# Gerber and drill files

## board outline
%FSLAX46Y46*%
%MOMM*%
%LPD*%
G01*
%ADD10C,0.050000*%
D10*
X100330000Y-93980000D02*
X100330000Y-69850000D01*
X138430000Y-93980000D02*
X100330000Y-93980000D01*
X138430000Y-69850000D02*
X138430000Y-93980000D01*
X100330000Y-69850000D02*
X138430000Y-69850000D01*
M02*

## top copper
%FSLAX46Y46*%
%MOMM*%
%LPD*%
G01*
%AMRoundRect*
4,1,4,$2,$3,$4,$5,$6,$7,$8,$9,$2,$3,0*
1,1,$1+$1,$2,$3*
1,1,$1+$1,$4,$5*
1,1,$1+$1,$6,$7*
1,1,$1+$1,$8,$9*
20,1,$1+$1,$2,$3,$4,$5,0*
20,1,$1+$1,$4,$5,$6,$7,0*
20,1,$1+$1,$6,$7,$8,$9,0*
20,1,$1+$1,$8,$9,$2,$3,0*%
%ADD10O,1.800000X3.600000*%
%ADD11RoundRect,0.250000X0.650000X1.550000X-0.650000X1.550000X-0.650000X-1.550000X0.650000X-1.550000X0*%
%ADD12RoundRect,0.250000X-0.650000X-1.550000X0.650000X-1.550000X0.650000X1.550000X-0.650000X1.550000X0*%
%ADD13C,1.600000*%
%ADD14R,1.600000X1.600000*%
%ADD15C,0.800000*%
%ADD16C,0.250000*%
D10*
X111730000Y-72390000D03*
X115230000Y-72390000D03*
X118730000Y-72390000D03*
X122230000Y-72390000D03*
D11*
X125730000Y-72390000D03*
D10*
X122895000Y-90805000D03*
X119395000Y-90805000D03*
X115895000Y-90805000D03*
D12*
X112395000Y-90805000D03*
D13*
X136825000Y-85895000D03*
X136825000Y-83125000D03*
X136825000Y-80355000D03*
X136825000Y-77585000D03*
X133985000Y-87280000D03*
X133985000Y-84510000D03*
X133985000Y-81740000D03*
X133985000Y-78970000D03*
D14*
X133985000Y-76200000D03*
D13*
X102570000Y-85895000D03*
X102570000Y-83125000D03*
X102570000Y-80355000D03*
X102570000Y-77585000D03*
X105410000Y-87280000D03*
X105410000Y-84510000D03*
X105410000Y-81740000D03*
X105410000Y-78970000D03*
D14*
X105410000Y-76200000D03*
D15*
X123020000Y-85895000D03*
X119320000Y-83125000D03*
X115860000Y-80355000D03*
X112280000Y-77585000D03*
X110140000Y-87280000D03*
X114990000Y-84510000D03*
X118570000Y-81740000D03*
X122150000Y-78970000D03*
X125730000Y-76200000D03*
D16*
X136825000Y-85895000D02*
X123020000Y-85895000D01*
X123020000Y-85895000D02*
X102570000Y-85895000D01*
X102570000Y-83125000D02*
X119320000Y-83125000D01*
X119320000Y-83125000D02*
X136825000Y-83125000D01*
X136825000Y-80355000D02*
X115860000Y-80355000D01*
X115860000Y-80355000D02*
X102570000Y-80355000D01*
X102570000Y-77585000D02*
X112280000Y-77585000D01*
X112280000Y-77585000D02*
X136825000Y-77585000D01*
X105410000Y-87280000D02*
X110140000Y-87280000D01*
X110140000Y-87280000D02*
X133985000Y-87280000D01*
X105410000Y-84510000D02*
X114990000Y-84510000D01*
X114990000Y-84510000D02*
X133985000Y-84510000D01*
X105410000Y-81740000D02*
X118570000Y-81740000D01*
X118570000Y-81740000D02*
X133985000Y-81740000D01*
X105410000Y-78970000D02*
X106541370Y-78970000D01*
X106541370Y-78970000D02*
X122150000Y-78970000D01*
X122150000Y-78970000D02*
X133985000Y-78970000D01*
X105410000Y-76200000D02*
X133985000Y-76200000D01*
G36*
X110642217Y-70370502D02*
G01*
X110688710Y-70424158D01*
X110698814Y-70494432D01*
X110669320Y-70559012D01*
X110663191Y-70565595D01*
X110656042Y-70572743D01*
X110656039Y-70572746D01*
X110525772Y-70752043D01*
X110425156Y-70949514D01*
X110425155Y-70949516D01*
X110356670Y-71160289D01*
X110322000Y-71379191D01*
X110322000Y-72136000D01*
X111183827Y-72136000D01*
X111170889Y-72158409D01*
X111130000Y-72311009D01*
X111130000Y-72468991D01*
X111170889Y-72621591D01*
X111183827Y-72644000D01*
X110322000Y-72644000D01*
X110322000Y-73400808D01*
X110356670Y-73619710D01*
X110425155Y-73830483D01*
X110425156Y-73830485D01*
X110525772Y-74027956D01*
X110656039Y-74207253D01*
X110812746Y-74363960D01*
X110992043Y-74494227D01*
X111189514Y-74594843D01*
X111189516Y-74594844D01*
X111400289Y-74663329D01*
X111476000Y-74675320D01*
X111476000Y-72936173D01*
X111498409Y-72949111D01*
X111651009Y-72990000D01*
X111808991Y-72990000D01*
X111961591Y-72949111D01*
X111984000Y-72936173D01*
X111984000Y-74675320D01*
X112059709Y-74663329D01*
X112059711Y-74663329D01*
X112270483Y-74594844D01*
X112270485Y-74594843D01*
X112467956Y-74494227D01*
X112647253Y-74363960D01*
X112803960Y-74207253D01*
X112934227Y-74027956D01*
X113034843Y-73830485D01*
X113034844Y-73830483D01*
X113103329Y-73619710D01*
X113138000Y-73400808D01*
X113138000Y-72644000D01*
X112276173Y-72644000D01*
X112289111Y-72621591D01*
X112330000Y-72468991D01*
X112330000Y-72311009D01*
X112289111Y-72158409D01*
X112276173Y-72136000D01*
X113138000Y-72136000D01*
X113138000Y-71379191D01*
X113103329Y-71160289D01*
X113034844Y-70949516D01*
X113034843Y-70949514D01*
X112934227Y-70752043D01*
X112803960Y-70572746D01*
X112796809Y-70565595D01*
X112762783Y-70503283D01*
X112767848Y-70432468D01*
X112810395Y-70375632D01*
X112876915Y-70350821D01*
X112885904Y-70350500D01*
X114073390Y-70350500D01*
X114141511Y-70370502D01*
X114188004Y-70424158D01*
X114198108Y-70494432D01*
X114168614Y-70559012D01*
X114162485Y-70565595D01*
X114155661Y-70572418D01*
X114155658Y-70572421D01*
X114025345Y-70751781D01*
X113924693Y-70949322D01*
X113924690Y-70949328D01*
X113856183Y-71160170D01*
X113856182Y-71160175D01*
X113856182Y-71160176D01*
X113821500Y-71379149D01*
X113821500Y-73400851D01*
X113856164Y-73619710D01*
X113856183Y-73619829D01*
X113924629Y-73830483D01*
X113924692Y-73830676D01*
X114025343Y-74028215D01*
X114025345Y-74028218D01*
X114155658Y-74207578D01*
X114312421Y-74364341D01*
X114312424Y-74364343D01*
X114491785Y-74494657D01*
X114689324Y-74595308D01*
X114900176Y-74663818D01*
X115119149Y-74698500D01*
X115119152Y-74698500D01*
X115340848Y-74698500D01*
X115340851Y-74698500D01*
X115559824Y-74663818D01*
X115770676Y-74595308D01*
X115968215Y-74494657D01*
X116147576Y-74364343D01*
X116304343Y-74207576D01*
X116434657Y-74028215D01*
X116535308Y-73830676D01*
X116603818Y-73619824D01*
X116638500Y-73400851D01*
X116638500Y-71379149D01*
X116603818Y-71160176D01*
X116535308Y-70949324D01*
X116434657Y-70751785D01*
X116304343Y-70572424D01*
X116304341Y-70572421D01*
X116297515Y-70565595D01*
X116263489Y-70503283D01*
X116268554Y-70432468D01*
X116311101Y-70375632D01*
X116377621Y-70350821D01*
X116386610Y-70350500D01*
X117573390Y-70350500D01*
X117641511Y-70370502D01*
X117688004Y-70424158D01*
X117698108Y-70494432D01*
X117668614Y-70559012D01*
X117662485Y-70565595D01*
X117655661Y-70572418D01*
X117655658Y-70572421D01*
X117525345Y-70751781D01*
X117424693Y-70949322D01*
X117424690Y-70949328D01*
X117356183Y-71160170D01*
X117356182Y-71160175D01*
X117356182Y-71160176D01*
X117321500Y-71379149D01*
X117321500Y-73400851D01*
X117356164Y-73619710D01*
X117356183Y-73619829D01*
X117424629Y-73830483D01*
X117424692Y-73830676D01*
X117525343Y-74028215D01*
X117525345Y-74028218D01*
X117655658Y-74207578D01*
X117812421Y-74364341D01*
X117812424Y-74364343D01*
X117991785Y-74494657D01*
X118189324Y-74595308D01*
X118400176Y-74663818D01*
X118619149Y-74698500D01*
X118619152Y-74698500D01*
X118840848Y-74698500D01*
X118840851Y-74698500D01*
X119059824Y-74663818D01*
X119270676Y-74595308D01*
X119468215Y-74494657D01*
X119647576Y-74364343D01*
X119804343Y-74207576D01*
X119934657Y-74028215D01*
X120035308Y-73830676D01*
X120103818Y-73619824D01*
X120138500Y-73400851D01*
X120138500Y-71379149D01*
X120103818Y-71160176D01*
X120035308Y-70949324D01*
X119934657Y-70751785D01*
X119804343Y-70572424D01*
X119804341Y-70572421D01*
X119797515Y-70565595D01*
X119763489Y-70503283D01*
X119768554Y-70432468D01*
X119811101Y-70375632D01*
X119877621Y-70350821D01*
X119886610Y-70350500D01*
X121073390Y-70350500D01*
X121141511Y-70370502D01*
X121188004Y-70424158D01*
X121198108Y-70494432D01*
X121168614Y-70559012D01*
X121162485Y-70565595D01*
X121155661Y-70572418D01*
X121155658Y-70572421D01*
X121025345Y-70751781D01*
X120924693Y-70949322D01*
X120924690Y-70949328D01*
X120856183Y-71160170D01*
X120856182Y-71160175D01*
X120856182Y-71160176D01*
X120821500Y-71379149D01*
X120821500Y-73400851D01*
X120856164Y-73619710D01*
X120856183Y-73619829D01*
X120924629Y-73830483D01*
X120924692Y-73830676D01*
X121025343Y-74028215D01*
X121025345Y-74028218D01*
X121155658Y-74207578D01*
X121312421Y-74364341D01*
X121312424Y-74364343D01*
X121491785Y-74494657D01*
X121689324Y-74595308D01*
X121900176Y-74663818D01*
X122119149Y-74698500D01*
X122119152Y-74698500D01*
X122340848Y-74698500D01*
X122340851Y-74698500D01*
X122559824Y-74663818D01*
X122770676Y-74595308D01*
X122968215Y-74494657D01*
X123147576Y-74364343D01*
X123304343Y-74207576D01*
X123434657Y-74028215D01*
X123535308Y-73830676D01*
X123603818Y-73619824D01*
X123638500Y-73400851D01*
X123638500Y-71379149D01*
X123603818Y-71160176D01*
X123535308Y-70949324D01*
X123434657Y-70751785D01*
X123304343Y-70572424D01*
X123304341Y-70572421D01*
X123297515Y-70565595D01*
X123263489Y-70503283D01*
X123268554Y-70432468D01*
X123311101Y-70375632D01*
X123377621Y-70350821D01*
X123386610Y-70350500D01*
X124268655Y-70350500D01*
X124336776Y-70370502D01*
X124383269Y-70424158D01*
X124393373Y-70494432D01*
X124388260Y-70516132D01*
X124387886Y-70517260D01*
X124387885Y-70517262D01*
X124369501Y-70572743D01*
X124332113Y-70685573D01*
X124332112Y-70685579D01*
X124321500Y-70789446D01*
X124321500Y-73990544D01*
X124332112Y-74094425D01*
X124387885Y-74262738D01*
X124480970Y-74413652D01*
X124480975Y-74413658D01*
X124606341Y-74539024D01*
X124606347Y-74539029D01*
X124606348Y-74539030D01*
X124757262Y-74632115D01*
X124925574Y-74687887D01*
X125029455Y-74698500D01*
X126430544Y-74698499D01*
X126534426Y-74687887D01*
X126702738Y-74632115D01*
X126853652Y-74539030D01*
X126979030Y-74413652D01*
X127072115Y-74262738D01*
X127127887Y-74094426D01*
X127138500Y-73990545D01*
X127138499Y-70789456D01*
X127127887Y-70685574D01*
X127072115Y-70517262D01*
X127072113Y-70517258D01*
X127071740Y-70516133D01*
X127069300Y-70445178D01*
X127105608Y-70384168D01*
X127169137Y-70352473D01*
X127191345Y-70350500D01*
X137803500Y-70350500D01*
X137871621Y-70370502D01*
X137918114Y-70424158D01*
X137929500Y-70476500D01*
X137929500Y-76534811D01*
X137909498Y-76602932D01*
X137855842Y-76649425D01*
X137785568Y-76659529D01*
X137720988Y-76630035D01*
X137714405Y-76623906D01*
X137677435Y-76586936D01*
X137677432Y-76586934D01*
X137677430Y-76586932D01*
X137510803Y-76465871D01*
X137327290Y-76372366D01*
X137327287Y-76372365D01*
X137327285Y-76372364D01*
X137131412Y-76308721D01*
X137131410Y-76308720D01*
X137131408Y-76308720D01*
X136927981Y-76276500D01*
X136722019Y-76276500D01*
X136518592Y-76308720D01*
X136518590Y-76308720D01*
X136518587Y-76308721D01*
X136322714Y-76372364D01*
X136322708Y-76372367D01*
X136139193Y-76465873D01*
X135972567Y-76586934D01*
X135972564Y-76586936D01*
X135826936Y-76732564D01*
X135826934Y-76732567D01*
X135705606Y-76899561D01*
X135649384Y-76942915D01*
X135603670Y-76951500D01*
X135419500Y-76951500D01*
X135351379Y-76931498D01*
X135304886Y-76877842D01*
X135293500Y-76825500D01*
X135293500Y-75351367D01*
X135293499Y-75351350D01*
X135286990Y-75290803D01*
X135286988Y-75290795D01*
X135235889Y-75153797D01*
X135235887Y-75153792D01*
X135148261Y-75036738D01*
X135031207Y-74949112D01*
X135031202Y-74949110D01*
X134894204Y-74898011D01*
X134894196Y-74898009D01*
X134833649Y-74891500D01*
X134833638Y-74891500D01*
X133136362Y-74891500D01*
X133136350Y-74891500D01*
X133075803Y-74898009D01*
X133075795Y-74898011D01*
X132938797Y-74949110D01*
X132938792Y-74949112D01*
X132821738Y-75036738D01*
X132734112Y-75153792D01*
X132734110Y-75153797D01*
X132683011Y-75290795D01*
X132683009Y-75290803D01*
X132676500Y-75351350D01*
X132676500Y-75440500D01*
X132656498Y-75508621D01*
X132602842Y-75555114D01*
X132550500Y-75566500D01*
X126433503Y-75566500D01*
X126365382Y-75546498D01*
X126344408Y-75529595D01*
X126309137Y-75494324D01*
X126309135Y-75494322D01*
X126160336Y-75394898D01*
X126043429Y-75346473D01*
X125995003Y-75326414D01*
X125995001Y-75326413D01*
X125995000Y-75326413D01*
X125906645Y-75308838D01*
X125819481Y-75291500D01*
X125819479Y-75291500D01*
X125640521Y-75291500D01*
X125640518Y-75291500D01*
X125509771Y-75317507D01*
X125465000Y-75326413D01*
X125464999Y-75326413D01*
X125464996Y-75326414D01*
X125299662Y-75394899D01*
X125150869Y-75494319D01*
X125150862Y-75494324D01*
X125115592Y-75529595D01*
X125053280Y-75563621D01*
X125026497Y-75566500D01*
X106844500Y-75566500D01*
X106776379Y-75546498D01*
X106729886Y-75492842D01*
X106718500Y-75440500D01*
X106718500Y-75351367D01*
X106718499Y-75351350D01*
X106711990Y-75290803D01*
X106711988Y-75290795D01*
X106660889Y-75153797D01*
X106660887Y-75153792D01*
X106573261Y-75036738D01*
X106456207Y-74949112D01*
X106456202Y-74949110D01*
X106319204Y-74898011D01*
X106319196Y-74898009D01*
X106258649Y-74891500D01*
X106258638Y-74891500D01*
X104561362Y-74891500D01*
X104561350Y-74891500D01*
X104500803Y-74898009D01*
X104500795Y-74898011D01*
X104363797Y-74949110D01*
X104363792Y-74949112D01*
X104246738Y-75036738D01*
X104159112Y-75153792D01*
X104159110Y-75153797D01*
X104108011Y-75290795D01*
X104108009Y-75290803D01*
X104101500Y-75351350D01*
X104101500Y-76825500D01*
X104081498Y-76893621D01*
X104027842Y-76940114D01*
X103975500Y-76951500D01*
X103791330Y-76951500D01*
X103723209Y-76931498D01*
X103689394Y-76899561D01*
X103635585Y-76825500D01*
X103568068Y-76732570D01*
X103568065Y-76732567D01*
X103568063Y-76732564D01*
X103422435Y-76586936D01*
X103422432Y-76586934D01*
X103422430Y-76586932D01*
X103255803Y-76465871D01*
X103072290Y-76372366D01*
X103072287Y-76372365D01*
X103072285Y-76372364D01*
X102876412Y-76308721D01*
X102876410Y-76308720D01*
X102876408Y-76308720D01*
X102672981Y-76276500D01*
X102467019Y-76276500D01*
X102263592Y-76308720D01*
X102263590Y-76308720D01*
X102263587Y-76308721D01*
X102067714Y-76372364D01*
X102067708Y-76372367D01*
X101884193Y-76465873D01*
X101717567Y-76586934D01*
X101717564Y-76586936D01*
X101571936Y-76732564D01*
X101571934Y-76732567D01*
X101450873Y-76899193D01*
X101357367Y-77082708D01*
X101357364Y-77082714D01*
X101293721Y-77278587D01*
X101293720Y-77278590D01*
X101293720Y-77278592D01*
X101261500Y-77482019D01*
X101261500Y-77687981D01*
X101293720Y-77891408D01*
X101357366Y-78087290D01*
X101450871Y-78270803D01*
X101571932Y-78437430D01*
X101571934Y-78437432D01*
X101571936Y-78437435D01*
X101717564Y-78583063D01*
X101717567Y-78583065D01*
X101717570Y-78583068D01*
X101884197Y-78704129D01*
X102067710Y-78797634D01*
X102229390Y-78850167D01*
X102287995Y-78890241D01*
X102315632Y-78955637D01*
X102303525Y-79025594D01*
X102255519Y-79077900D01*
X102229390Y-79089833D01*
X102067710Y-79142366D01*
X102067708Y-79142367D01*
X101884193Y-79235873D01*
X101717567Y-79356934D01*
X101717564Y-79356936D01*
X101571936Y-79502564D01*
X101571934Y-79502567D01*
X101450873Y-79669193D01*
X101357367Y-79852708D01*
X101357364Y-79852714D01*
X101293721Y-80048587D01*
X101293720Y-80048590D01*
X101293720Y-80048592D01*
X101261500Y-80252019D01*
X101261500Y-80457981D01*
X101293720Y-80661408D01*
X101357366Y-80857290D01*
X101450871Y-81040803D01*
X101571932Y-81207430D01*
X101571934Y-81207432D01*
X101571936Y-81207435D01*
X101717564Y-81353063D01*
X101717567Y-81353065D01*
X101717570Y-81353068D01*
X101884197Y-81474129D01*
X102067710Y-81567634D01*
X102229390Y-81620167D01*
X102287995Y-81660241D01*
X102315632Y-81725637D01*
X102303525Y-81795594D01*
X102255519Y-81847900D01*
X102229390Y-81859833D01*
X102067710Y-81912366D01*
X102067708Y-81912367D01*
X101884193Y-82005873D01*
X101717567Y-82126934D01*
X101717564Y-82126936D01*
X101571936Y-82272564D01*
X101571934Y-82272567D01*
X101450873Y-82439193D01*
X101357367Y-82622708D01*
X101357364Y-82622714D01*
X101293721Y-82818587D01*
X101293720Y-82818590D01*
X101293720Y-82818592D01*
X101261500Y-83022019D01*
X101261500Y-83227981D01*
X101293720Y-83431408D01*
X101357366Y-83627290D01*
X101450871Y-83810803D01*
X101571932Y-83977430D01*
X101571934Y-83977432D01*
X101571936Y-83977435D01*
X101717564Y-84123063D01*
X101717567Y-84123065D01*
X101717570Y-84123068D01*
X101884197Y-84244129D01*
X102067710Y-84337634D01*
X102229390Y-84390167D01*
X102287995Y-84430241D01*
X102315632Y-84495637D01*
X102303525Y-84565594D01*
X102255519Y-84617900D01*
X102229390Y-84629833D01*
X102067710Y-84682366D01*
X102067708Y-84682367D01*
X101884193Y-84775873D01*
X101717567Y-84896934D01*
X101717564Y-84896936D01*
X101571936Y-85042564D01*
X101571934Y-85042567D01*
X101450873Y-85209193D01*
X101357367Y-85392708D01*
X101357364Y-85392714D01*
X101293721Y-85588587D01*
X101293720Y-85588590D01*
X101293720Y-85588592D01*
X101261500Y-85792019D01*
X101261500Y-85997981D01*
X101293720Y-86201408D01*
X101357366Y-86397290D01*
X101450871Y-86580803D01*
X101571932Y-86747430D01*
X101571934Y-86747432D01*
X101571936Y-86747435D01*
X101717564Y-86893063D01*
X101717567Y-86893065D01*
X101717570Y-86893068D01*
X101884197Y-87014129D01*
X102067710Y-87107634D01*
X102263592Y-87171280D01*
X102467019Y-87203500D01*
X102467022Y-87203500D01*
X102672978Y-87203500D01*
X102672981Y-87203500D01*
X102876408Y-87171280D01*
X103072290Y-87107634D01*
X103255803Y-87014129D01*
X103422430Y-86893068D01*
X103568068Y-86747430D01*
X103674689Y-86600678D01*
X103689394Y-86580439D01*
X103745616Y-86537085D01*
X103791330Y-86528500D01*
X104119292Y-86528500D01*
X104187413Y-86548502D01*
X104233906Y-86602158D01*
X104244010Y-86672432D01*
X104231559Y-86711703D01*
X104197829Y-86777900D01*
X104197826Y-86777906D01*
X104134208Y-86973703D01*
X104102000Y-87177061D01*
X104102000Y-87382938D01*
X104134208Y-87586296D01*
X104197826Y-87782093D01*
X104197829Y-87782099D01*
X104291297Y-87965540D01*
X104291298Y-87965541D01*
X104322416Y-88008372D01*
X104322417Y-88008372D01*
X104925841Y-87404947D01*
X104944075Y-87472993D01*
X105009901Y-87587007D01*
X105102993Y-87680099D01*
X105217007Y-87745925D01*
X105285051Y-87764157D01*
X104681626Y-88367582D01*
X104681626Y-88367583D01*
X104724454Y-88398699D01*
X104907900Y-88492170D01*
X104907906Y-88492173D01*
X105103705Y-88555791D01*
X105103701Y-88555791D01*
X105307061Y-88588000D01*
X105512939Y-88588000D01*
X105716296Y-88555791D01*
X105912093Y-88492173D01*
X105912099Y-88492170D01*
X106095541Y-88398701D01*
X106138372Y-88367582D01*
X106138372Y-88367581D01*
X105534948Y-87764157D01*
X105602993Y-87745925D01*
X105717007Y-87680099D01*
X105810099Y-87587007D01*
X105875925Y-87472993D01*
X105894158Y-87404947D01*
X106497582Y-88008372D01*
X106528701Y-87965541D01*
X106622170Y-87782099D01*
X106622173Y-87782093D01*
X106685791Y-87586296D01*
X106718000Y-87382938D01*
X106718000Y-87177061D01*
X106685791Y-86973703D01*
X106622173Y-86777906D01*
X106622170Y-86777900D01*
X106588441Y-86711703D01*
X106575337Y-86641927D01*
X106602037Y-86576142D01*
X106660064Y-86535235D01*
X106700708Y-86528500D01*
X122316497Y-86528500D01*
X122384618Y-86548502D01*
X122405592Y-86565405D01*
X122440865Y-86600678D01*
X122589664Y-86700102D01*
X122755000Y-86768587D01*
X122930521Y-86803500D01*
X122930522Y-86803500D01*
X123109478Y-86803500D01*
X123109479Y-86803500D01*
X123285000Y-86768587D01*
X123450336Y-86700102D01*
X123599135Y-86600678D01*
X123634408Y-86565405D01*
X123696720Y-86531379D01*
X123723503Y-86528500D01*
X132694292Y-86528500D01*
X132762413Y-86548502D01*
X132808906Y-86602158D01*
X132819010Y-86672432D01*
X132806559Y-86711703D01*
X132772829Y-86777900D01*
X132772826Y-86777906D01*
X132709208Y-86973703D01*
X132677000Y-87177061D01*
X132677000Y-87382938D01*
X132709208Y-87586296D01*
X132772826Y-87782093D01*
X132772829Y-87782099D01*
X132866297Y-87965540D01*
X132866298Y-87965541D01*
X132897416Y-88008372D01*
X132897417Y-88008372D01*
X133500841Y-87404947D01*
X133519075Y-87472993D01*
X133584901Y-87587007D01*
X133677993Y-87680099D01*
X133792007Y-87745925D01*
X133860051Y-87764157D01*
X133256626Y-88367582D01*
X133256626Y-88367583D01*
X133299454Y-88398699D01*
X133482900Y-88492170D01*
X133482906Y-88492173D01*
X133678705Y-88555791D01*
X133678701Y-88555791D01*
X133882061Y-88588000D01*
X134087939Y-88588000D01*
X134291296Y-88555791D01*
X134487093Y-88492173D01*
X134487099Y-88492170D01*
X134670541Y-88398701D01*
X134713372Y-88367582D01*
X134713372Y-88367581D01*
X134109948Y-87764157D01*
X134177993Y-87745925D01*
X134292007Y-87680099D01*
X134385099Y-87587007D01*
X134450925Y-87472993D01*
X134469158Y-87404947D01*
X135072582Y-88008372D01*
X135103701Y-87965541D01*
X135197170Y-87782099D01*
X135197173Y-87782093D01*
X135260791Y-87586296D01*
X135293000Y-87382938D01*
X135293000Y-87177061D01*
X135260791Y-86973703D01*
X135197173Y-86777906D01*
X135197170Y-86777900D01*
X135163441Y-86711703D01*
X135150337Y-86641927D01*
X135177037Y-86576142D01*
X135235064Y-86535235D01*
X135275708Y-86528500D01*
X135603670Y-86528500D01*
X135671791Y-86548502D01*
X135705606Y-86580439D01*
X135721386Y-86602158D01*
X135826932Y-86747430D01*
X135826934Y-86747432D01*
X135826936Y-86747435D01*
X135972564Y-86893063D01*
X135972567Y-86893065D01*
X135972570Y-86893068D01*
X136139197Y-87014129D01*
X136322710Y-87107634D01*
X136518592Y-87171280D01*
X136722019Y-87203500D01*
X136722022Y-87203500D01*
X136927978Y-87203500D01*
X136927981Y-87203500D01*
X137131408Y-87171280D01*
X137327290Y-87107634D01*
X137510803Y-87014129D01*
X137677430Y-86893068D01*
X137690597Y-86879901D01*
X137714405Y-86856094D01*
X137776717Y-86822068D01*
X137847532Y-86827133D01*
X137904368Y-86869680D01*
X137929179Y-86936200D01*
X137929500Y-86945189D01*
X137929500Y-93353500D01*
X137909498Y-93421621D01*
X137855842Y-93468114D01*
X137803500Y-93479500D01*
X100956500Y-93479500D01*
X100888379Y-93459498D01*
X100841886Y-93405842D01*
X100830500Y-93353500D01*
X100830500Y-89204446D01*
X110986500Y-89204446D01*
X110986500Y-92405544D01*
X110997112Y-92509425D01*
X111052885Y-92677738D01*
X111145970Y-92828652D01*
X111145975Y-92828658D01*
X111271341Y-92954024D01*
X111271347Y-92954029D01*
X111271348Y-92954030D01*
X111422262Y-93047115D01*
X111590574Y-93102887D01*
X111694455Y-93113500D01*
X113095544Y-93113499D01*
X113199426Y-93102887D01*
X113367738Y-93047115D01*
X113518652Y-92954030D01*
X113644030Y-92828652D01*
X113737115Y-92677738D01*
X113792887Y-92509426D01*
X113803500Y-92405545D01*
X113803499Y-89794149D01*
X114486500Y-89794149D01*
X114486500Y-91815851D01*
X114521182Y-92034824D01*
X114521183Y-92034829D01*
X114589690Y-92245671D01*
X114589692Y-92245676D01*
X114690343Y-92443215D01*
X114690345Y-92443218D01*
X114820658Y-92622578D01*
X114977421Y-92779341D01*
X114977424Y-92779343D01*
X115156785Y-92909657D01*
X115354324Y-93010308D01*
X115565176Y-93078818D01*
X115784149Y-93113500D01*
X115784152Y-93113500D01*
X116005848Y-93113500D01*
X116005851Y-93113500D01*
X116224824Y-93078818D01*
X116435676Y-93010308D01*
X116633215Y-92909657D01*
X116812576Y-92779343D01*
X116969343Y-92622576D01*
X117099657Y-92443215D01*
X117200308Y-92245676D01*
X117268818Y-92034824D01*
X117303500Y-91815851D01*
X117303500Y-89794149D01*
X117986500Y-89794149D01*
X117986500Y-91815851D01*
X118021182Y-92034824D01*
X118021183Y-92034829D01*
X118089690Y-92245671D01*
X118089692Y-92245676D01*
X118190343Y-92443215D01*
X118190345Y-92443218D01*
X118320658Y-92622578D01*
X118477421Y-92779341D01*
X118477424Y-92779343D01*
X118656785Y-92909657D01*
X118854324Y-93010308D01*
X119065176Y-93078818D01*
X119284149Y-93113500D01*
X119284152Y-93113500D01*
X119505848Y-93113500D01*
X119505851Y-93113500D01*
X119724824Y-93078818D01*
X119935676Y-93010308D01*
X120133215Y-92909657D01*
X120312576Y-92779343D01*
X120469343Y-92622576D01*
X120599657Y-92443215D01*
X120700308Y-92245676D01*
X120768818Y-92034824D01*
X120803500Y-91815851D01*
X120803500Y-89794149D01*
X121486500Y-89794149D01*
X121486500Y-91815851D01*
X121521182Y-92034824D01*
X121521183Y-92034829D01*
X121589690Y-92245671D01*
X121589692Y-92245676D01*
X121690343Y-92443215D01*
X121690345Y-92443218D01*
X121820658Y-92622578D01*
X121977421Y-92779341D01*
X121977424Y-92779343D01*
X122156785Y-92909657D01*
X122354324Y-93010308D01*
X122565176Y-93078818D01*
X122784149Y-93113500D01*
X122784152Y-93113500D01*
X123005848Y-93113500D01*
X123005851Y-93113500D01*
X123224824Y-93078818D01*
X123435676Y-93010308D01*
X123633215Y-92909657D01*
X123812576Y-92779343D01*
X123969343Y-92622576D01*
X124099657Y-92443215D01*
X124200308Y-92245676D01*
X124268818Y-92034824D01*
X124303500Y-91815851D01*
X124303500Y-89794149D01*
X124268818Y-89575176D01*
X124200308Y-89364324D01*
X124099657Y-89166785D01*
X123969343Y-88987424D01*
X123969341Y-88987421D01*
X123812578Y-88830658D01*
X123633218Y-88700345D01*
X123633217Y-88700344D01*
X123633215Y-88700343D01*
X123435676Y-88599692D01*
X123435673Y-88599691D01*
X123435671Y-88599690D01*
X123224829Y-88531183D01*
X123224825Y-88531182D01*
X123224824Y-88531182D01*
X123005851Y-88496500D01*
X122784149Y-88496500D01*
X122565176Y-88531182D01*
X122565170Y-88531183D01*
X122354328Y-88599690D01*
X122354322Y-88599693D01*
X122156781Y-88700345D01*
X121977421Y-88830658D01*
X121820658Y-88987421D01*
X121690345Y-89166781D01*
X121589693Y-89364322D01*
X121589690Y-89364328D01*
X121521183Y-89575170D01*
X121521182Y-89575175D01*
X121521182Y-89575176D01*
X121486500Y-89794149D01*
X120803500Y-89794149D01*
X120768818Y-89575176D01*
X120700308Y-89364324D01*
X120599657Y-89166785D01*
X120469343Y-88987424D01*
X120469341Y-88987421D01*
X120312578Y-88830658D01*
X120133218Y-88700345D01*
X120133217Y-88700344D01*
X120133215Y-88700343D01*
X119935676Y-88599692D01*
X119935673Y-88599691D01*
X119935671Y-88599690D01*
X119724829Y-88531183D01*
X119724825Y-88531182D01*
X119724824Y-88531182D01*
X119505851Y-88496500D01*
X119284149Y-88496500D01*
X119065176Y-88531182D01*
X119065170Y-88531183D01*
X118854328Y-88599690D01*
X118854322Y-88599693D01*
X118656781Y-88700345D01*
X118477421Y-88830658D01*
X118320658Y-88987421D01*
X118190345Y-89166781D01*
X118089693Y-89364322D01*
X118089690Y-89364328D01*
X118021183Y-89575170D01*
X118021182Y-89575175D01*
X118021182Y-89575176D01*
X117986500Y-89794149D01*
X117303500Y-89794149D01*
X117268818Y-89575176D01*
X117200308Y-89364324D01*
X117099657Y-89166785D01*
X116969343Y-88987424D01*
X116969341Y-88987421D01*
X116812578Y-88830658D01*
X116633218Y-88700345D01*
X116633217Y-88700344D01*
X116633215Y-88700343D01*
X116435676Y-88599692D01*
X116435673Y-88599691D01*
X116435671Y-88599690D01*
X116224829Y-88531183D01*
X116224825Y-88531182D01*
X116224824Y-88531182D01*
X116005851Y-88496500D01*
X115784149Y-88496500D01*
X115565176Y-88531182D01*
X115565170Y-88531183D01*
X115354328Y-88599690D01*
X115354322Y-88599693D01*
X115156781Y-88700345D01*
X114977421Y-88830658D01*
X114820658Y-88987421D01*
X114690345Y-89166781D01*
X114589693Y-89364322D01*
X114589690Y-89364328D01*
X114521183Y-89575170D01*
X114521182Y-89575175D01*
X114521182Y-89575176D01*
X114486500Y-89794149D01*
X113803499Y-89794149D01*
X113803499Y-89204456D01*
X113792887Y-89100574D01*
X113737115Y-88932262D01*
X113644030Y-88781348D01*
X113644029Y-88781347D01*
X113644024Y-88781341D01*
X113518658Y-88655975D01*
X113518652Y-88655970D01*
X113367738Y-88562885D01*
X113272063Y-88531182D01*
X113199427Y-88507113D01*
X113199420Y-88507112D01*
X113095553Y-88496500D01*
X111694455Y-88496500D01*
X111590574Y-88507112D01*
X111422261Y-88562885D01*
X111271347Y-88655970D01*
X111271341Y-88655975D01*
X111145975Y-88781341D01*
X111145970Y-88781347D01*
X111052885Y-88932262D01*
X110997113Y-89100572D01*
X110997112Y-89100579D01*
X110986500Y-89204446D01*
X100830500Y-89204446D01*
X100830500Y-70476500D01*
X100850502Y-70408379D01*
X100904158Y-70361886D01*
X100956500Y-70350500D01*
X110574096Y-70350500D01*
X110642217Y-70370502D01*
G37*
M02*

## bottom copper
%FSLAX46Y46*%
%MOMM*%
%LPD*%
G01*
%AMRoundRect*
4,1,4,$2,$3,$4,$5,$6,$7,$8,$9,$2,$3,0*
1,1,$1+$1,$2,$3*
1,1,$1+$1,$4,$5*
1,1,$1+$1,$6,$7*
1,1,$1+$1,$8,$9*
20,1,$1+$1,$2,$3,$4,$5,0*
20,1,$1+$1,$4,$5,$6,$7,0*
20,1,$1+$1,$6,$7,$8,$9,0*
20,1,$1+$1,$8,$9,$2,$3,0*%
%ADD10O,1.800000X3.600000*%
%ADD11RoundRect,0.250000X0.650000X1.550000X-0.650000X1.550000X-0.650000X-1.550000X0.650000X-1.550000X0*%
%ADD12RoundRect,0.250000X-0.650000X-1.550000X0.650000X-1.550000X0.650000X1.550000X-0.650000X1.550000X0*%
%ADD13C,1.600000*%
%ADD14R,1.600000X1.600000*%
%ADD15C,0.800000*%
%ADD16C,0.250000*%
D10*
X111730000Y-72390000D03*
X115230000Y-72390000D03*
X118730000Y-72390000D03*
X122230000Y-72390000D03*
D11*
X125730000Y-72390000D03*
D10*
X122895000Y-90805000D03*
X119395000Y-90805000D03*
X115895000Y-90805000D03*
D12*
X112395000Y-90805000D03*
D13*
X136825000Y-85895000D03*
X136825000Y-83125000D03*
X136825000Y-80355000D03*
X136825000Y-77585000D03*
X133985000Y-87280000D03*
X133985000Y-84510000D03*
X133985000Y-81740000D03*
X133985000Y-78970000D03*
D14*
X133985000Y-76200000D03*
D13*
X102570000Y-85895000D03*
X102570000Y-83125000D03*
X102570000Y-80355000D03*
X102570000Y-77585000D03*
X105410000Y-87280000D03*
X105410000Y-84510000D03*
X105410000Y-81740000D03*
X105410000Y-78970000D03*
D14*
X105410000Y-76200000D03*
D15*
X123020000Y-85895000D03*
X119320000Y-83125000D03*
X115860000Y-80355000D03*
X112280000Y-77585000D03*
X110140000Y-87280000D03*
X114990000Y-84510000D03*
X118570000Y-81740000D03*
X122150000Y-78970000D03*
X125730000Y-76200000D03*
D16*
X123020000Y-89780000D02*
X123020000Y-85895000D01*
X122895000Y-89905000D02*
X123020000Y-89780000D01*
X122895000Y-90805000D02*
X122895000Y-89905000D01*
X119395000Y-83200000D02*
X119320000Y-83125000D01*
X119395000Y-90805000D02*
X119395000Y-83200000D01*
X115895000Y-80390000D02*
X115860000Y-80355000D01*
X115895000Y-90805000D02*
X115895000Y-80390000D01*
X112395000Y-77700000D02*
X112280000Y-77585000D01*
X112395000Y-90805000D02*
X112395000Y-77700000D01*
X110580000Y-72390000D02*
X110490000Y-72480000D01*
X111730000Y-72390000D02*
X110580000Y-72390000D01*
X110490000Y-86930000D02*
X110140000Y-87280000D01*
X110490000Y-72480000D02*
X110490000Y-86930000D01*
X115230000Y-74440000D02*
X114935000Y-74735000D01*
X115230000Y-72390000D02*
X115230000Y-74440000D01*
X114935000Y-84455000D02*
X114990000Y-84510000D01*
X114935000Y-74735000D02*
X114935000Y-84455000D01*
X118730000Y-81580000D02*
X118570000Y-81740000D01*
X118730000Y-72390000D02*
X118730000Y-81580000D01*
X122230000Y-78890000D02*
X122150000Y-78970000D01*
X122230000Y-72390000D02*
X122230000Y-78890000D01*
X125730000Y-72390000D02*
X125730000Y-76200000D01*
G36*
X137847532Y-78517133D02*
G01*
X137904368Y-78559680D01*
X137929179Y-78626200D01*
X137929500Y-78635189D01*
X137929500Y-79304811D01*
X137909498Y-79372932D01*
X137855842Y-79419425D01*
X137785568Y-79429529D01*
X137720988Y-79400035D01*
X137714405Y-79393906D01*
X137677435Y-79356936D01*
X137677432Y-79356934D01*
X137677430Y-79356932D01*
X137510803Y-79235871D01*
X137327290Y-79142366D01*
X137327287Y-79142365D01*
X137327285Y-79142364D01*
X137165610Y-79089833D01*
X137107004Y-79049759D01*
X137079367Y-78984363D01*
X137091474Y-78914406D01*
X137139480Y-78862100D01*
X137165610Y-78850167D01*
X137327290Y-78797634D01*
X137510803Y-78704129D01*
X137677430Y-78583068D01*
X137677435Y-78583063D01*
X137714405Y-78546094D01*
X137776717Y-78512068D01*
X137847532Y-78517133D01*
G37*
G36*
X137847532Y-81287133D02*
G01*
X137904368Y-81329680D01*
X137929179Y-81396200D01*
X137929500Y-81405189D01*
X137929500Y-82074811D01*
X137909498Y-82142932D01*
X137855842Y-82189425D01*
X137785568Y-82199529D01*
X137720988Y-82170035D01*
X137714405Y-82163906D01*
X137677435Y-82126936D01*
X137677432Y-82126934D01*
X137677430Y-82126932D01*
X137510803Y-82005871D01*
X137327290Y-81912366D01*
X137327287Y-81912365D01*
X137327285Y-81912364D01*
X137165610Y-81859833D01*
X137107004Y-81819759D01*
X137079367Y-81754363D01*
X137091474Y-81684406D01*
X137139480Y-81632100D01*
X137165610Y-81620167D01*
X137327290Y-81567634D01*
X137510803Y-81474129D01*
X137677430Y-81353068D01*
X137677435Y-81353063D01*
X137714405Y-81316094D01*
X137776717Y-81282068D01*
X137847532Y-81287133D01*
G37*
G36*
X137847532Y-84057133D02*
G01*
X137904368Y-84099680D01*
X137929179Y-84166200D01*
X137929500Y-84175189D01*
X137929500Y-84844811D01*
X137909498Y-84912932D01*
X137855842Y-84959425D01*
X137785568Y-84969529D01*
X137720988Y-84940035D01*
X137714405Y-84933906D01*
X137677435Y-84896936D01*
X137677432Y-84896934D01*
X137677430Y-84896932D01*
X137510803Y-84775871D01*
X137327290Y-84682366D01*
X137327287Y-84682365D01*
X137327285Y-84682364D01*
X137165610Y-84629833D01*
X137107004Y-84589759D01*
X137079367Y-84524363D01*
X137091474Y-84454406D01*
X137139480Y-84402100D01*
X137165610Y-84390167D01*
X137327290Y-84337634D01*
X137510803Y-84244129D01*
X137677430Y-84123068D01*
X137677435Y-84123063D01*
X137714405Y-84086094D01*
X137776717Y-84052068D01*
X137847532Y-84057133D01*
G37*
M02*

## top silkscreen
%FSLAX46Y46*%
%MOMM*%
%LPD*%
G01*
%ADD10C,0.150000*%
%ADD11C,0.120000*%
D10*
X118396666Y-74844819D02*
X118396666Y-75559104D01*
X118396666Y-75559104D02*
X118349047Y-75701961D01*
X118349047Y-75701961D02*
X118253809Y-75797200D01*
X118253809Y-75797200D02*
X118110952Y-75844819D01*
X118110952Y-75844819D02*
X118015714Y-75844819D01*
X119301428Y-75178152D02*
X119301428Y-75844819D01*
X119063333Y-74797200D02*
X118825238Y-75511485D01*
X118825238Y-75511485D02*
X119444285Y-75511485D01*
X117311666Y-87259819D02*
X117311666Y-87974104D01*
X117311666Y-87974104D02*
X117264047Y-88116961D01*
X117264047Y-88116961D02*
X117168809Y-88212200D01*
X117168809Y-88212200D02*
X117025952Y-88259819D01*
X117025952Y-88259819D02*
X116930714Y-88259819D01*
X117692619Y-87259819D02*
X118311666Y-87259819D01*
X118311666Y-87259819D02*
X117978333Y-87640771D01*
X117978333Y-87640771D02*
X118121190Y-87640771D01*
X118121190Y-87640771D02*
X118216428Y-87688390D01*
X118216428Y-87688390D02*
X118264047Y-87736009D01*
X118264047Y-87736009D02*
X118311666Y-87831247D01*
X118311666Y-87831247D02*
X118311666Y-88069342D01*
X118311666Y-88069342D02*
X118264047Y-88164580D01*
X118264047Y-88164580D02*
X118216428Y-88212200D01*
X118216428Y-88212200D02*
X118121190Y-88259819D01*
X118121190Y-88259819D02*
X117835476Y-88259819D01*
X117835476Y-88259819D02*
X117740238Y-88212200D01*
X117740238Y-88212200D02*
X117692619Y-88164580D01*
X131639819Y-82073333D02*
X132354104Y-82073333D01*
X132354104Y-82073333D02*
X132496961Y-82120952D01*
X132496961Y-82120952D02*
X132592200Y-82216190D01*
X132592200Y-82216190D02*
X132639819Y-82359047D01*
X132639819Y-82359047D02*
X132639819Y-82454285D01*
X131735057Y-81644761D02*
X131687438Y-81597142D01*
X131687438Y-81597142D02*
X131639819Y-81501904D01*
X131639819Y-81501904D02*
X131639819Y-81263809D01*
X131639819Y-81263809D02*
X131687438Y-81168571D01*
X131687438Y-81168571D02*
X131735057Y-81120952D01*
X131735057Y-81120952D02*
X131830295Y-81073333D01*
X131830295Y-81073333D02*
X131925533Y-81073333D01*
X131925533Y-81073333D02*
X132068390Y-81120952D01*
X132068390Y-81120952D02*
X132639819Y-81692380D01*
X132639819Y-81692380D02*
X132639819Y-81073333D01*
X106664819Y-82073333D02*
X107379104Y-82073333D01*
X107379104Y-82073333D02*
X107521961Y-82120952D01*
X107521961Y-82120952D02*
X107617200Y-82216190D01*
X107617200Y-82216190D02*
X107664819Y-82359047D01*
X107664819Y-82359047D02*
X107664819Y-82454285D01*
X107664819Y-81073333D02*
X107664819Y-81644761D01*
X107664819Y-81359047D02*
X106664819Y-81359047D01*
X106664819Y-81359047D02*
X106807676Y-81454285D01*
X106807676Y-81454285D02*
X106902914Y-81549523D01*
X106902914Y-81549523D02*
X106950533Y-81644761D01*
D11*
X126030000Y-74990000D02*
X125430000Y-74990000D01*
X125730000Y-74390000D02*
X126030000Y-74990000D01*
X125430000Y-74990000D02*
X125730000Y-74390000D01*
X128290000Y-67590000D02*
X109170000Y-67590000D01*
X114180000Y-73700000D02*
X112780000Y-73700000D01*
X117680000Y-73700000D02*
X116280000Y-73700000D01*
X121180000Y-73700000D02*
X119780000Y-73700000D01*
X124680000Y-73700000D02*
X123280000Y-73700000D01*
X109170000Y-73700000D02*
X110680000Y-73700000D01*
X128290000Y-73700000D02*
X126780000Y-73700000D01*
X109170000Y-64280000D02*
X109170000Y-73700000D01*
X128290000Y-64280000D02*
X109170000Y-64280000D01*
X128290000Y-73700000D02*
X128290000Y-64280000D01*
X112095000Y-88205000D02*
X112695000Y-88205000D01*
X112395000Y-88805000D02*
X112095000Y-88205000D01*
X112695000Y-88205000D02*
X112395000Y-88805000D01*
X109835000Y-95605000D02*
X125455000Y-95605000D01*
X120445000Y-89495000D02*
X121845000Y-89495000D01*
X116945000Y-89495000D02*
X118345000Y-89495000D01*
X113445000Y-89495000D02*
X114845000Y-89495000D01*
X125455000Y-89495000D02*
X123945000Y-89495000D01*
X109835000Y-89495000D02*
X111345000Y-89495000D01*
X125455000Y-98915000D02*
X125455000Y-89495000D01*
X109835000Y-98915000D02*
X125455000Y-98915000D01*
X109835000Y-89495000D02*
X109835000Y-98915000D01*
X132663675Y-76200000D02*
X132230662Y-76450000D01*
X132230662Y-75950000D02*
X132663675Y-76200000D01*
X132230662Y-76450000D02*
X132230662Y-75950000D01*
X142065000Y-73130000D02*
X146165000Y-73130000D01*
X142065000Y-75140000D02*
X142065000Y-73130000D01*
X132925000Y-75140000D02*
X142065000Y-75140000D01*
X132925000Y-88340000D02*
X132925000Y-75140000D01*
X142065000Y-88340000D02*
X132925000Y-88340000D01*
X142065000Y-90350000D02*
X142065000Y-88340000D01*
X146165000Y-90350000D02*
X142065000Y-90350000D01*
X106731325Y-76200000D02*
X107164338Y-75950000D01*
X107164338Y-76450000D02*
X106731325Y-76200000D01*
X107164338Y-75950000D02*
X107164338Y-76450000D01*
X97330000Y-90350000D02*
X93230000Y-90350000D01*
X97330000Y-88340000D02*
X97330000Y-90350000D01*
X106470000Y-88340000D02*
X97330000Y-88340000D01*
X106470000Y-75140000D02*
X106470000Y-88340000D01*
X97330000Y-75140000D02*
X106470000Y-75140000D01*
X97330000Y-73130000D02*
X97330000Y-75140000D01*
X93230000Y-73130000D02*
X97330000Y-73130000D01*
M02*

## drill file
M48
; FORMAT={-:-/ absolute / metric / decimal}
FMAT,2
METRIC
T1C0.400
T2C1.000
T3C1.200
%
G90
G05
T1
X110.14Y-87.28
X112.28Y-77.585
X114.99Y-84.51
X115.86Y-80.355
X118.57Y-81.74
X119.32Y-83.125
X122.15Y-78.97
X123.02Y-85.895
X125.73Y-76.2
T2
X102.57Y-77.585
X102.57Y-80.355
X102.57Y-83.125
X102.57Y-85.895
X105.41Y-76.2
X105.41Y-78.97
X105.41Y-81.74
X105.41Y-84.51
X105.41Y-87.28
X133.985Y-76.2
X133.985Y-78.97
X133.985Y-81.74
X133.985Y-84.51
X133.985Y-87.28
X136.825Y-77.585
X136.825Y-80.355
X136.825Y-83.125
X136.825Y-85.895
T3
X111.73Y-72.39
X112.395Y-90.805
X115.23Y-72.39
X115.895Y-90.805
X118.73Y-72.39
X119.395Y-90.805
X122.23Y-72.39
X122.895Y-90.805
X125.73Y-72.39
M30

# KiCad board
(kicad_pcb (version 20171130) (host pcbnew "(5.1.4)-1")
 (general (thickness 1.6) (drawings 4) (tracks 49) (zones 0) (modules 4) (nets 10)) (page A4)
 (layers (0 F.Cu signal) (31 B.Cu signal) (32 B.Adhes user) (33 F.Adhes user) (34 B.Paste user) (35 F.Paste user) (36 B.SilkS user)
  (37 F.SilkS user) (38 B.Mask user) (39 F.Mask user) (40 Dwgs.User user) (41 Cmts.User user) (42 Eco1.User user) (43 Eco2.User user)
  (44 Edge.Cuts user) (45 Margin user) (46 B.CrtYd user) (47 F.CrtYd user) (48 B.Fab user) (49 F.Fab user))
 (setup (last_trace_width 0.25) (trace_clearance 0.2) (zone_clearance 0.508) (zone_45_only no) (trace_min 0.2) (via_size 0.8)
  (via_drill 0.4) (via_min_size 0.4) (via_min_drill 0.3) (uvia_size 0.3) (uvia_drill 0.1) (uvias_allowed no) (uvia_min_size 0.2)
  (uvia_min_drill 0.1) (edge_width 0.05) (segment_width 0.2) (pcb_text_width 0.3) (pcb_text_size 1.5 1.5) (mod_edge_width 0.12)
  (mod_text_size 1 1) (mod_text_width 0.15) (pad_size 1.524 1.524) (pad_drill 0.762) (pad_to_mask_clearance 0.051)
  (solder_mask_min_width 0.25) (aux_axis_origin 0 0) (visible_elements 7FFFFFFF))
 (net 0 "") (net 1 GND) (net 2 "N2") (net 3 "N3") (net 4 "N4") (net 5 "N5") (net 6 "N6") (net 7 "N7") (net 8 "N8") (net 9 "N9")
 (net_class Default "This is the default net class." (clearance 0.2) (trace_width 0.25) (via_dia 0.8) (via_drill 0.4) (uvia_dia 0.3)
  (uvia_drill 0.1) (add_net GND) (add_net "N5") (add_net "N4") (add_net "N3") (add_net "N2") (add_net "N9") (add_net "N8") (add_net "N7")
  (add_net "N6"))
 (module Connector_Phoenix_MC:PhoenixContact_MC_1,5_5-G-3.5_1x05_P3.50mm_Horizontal (layer F.Cu) (at 125.73 72.39 180)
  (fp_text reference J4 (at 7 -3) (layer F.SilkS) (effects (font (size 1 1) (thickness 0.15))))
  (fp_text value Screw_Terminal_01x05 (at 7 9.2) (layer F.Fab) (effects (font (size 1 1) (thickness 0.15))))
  (fp_line (start -0.3 -2.6) (end 0.3 -2.6) (layer F.SilkS) (width 0.12))
  (fp_line (start 0 -2) (end -0.3 -2.6) (layer F.SilkS) (width 0.12))
  (fp_line (start 0.3 -2.6) (end 0 -2) (layer F.SilkS) (width 0.12))
  (fp_line (start -2.56 4.8) (end 16.56 4.8) (layer F.SilkS) (width 0.12))
  (fp_line (start 11.55 -1.31) (end 12.95 -1.31) (layer F.SilkS) (width 0.12))
  (fp_line (start 8.05 -1.31) (end 9.45 -1.31) (layer F.SilkS) (width 0.12))
  (fp_line (start 4.55 -1.31) (end 5.95 -1.31) (layer F.SilkS) (width 0.12))
  (fp_line (start 1.05 -1.31) (end 2.45 -1.31) (layer F.SilkS) (width 0.12))
  (fp_line (start 16.56 -1.31) (end 15.05 -1.31) (layer F.SilkS) (width 0.12))
  (fp_line (start -2.56 -1.31) (end -1.05 -1.31) (layer F.SilkS) (width 0.12))
  (fp_line (start 16.56 8.11) (end 16.56 -1.31) (layer F.SilkS) (width 0.12))
  (fp_line (start -2.56 8.11) (end 16.56 8.11) (layer F.SilkS) (width 0.12))
  (fp_line (start -2.56 -1.31) (end -2.56 8.11) (layer F.SilkS) (width 0.12))
  (pad 5 thru_hole oval (at 14 0 180) (size 1.8 3.6) (drill 1.2) (layers *.Cu *.Mask) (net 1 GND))
  (pad 4 thru_hole oval (at 10.5 0 180) (size 1.8 3.6) (drill 1.2) (layers *.Cu *.Mask) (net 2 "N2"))
  (pad 3 thru_hole oval (at 7 0 180) (size 1.8 3.6) (drill 1.2) (layers *.Cu *.Mask) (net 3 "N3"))
  (pad 2 thru_hole oval (at 3.5 0 180) (size 1.8 3.6) (drill 1.2) (layers *.Cu *.Mask) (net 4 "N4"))
  (pad 1 thru_hole roundrect (at 0 0 180) (size 1.8 3.6) (drill 1.2) (layers *.Cu *.Mask) (roundrect_rratio 0.138889) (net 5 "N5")))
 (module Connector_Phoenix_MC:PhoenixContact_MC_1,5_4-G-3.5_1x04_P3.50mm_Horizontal (layer F.Cu) (at 112.395 90.805)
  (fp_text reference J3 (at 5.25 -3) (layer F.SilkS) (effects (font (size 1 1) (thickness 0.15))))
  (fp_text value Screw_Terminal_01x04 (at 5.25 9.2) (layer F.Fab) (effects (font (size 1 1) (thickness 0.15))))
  (fp_line (start -0.3 -2.6) (end 0.3 -2.6) (layer F.SilkS) (width 0.12))
  (fp_line (start 0 -2) (end -0.3 -2.6) (layer F.SilkS) (width 0.12))
  (fp_line (start 0.3 -2.6) (end 0 -2) (layer F.SilkS) (width 0.12))
  (fp_line (start -2.56 4.8) (end 13.06 4.8) (layer F.SilkS) (width 0.12))
  (fp_line (start 8.05 -1.31) (end 9.45 -1.31) (layer F.SilkS) (width 0.12))
  (fp_line (start 4.55 -1.31) (end 5.95 -1.31) (layer F.SilkS) (width 0.12))
  (fp_line (start 1.05 -1.31) (end 2.45 -1.31) (layer F.SilkS) (width 0.12))
  (fp_line (start 13.06 -1.31) (end 11.55 -1.31) (layer F.SilkS) (width 0.12))
  (fp_line (start -2.56 -1.31) (end -1.05 -1.31) (layer F.SilkS) (width 0.12))
  (fp_line (start 13.06 8.11) (end 13.06 -1.31) (layer F.SilkS) (width 0.12))
  (fp_line (start -2.56 8.11) (end 13.06 8.11) (layer F.SilkS) (width 0.12))
  (fp_line (start -2.56 -1.31) (end -2.56 8.11) (layer F.SilkS) (width 0.12))
  (pad 4 thru_hole oval (at 10.5 0) (size 1.8 3.6) (drill 1.2) (layers *.Cu *.Mask) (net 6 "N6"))
  (pad 3 thru_hole oval (at 7 0) (size 1.8 3.6) (drill 1.2) (layers *.Cu *.Mask) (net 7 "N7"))
  (pad 2 thru_hole oval (at 3.5 0) (size 1.8 3.6) (drill 1.2) (layers *.Cu *.Mask) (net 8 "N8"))
  (pad 1 thru_hole roundrect (at 0 0) (size 1.8 3.6) (drill 1.2) (layers *.Cu *.Mask) (roundrect_rratio 0.138889) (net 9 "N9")))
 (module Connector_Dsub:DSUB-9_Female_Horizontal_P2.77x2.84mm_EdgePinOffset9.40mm (layer F.Cu) (at 133.985 76.2 90)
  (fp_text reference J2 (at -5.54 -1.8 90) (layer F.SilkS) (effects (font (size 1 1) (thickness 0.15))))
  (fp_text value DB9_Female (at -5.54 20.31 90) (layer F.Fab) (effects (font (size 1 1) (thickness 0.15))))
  (fp_line (start 0 -1.321325) (end -0.25 -1.754338) (layer F.SilkS) (width 0.12))
  (fp_line (start 0.25 -1.754338) (end 0 -1.321325) (layer F.SilkS) (width 0.12))
  (fp_line (start -0.25 -1.754338) (end 0.25 -1.754338) (layer F.SilkS) (width 0.12))
  (fp_line (start 3.07 8.08) (end 3.07 12.18) (layer F.SilkS) (width 0.12))
  (fp_line (start 1.06 8.08) (end 3.07 8.08) (layer F.SilkS) (width 0.12))
  (fp_line (start 1.06 -1.06) (end 1.06 8.08) (layer F.SilkS) (width 0.12))
  (fp_line (start -12.14 -1.06) (end 1.06 -1.06) (layer F.SilkS) (width 0.12))
  (fp_line (start -12.14 8.08) (end -12.14 -1.06) (layer F.SilkS) (width 0.12))
  (fp_line (start -14.15 8.08) (end -12.14 8.08) (layer F.SilkS) (width 0.12))
  (fp_line (start -14.15 12.18) (end -14.15 8.08) (layer F.SilkS) (width 0.12))
  (pad 9 thru_hole circle (at -9.695 2.84 90) (size 1.6 1.6) (drill 1) (layers *.Cu *.Mask) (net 6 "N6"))
  (pad 8 thru_hole circle (at -6.925 2.84 90) (size 1.6 1.6) (drill 1) (layers *.Cu *.Mask) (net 7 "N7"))
  (pad 7 thru_hole circle (at -4.155 2.84 90) (size 1.6 1.6) (drill 1) (layers *.Cu *.Mask) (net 8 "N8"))
  (pad 6 thru_hole circle (at -1.385 2.84 90) (size 1.6 1.6) (drill 1) (layers *.Cu *.Mask) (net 9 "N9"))
  (pad 5 thru_hole circle (at -11.08 0 90) (size 1.6 1.6) (drill 1) (layers *.Cu *.Mask) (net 1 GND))
  (pad 4 thru_hole circle (at -8.31 0 90) (size 1.6 1.6) (drill 1) (layers *.Cu *.Mask) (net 2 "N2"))
  (pad 3 thru_hole circle (at -5.54 0 90) (size 1.6 1.6) (drill 1) (layers *.Cu *.Mask) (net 3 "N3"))
  (pad 2 thru_hole circle (at -2.77 0 90) (size 1.6 1.6) (drill 1) (layers *.Cu *.Mask) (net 4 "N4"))
  (pad 1 thru_hole rect (at 0 0 90) (size 1.6 1.6) (drill 1) (layers *.Cu *.Mask) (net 5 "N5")))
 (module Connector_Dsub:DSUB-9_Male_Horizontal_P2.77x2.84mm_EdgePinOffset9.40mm (layer F.Cu) (at 105.41 76.2 270)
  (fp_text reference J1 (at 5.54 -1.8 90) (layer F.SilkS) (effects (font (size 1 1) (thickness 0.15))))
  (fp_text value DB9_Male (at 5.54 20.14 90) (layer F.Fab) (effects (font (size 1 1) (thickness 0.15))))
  (fp_line (start 0 -1.321325) (end -0.25 -1.754338) (layer F.SilkS) (width 0.12))
  (fp_line (start 0.25 -1.754338) (end 0 -1.321325) (layer F.SilkS) (width 0.12))
  (fp_line (start -0.25 -1.754338) (end 0.25 -1.754338) (layer F.SilkS) (width 0.12))
  (fp_line (start 14.15 8.08) (end 14.15 12.18) (layer F.SilkS) (width 0.12))
  (fp_line (start 12.14 8.08) (end 14.15 8.08) (layer F.SilkS) (width 0.12))
  (fp_line (start 12.14 -1.06) (end 12.14 8.08) (layer F.SilkS) (width 0.12))
  (fp_line (start -1.06 -1.06) (end 12.14 -1.06) (layer F.SilkS) (width 0.12))
  (fp_line (start -1.06 8.08) (end -1.06 -1.06) (layer F.SilkS) (width 0.12))
  (fp_line (start -3.07 8.08) (end -1.06 8.08) (layer F.SilkS) (width 0.12))
  (fp_line (start -3.07 12.18) (end -3.07 8.08) (layer F.SilkS) (width 0.12))
  (pad 9 thru_hole circle (at 9.695 2.84 270) (size 1.6 1.6) (drill 1) (layers *.Cu *.Mask) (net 6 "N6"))
  (pad 8 thru_hole circle (at 6.925 2.84 270) (size 1.6 1.6) (drill 1) (layers *.Cu *.Mask) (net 7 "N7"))
  (pad 7 thru_hole circle (at 4.155 2.84 270) (size 1.6 1.6) (drill 1) (layers *.Cu *.Mask) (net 8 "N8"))
  (pad 6 thru_hole circle (at 1.385 2.84 270) (size 1.6 1.6) (drill 1) (layers *.Cu *.Mask) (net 9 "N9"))
  (pad 5 thru_hole circle (at 11.08 0 270) (size 1.6 1.6) (drill 1) (layers *.Cu *.Mask) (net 1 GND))
  (pad 4 thru_hole circle (at 8.31 0 270) (size 1.6 1.6) (drill 1) (layers *.Cu *.Mask) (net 2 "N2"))
  (pad 3 thru_hole circle (at 5.54 0 270) (size 1.6 1.6) (drill 1) (layers *.Cu *.Mask) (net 3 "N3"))
  (pad 2 thru_hole circle (at 2.77 0 270) (size 1.6 1.6) (drill 1) (layers *.Cu *.Mask) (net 4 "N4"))
  (pad 1 thru_hole rect (at 0 0 270) (size 1.6 1.6) (drill 1) (layers *.Cu *.Mask) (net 5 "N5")))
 (gr_line (start 100.33 93.98) (end 100.33 69.85) (layer Edge.Cuts) (width 0.05))
 (gr_line (start 138.43 93.98) (end 100.33 93.98) (layer Edge.Cuts) (width 0.05))
 (gr_line (start 138.43 69.85) (end 138.43 93.98) (layer Edge.Cuts) (width 0.05))
 (gr_line (start 100.33 69.85) (end 138.43 69.85) (layer Edge.Cuts) (width 0.05))
 (via (at 123.02 85.895) (size 0.8) (drill 0.4) (layers F.Cu B.Cu) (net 6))
 (segment (start 123.02 89.78) (end 123.02 85.895) (width 0.25) (layer B.Cu) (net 6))
 (segment (start 122.895 89.905) (end 123.02 89.78) (width 0.25) (layer B.Cu) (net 6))
 (segment (start 122.895 90.805) (end 122.895 89.905) (width 0.25) (layer B.Cu) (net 6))
 (segment (start 136.825 85.895) (end 123.02 85.895) (width 0.25) (layer F.Cu) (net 6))
 (segment (start 123.02 85.895) (end 102.57 85.895) (width 0.25) (layer F.Cu) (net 6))
 (via (at 119.32 83.125) (size 0.8) (drill 0.4) (layers F.Cu B.Cu) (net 7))
 (segment (start 119.395 83.2) (end 119.32 83.125) (width 0.25) (layer B.Cu) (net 7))
 (segment (start 119.395 90.805) (end 119.395 83.2) (width 0.25) (layer B.Cu) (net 7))
 (segment (start 102.57 83.125) (end 119.32 83.125) (width 0.25) (layer F.Cu) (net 7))
 (segment (start 119.32 83.125) (end 136.825 83.125) (width 0.25) (layer F.Cu) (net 7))
 (via (at 115.86 80.355) (size 0.8) (drill 0.4) (layers F.Cu B.Cu) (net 8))
 (segment (start 115.895 80.39) (end 115.86 80.355) (width 0.25) (layer B.Cu) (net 8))
 (segment (start 115.895 90.805) (end 115.895 80.39) (width 0.25) (layer B.Cu) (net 8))
 (segment (start 136.825 80.355) (end 115.86 80.355) (width 0.25) (layer F.Cu) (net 8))
 (segment (start 115.86 80.355) (end 102.57 80.355) (width 0.25) (layer F.Cu) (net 8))
 (via (at 112.28 77.585) (size 0.8) (drill 0.4) (layers F.Cu B.Cu) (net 9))
 (segment (start 112.395 77.7) (end 112.28 77.585) (width 0.25) (layer B.Cu) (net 9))
 (segment (start 112.395 90.805) (end 112.395 77.7) (width 0.25) (layer B.Cu) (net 9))
 (segment (start 102.57 77.585) (end 112.28 77.585) (width 0.25) (layer F.Cu) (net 9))
 (segment (start 112.28 77.585) (end 136.825 77.585) (width 0.25) (layer F.Cu) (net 9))
 (segment (start 110.58 72.39) (end 110.49 72.48) (width 0.25) (layer B.Cu) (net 1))
 (segment (start 111.73 72.39) (end 110.58 72.39) (width 0.25) (layer B.Cu) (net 1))
 (via (at 110.14 87.28) (size 0.8) (drill 0.4) (layers F.Cu B.Cu) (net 1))
 (segment (start 110.49 86.93) (end 110.14 87.28) (width 0.25) (layer B.Cu) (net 1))
 (segment (start 110.49 72.48) (end 110.49 86.93) (width 0.25) (layer B.Cu) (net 1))
 (segment (start 105.41 87.28) (end 110.14 87.28) (width 0.25) (layer F.Cu) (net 1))
 (segment (start 110.14 87.28) (end 133.985 87.28) (width 0.25) (layer F.Cu) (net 1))
 (segment (start 115.23 74.44) (end 114.935 74.735) (width 0.25) (layer B.Cu) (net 2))
 (segment (start 115.23 72.39) (end 115.23 74.44) (width 0.25) (layer B.Cu) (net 2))
 (via (at 114.99 84.51) (size 0.8) (drill 0.4) (layers F.Cu B.Cu) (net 2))
 (segment (start 114.935 84.455) (end 114.99 84.51) (width 0.25) (layer B.Cu) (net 2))
 (segment (start 114.935 74.735) (end 114.935 84.455) (width 0.25) (layer B.Cu) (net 2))
 (segment (start 105.41 84.51) (end 114.99 84.51) (width 0.25) (layer F.Cu) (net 2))
 (segment (start 114.99 84.51) (end 133.985 84.51) (width 0.25) (layer F.Cu) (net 2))
 (via (at 118.57 81.74) (size 0.8) (drill 0.4) (layers F.Cu B.Cu) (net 3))
 (segment (start 118.73 81.58) (end 118.57 81.74) (width 0.25) (layer B.Cu) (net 3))
 (segment (start 118.73 72.39) (end 118.73 81.58) (width 0.25) (layer B.Cu) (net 3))
 (segment (start 105.41 81.74) (end 118.57 81.74) (width 0.25) (layer F.Cu) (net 3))
 (segment (start 118.57 81.74) (end 133.985 81.74) (width 0.25) (layer F.Cu) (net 3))
 (segment (start 105.41 78.97) (end 106.54137 78.97) (width 0.25) (layer F.Cu) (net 4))
 (via (at 122.15 78.97) (size 0.8) (drill 0.4) (layers F.Cu B.Cu) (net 4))
 (segment (start 122.23 78.89) (end 122.15 78.97) (width 0.25) (layer B.Cu) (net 4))
 (segment (start 122.23 72.39) (end 122.23 78.89) (width 0.25) (layer B.Cu) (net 4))
 (segment (start 106.54137 78.97) (end 122.15 78.97) (width 0.25) (layer F.Cu) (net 4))
 (segment (start 122.15 78.97) (end 133.985 78.97) (width 0.25) (layer F.Cu) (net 4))
 (segment (start 105.41 76.2) (end 133.985 76.2) (width 0.25) (layer F.Cu) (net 5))
 (via (at 125.73 76.2) (size 0.8) (drill 0.4) (layers F.Cu B.Cu) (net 5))
 (segment (start 125.73 72.39) (end 125.73 76.2) (width 0.25) (layer B.Cu) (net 5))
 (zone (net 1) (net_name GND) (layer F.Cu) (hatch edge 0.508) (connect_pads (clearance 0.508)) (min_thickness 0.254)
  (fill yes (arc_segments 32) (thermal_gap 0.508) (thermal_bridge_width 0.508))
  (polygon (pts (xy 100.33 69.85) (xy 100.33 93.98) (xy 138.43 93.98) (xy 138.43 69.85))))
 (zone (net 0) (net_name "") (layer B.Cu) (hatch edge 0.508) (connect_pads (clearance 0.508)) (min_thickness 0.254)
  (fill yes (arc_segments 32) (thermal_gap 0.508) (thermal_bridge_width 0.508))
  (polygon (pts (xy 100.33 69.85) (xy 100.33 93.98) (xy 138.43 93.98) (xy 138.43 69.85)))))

